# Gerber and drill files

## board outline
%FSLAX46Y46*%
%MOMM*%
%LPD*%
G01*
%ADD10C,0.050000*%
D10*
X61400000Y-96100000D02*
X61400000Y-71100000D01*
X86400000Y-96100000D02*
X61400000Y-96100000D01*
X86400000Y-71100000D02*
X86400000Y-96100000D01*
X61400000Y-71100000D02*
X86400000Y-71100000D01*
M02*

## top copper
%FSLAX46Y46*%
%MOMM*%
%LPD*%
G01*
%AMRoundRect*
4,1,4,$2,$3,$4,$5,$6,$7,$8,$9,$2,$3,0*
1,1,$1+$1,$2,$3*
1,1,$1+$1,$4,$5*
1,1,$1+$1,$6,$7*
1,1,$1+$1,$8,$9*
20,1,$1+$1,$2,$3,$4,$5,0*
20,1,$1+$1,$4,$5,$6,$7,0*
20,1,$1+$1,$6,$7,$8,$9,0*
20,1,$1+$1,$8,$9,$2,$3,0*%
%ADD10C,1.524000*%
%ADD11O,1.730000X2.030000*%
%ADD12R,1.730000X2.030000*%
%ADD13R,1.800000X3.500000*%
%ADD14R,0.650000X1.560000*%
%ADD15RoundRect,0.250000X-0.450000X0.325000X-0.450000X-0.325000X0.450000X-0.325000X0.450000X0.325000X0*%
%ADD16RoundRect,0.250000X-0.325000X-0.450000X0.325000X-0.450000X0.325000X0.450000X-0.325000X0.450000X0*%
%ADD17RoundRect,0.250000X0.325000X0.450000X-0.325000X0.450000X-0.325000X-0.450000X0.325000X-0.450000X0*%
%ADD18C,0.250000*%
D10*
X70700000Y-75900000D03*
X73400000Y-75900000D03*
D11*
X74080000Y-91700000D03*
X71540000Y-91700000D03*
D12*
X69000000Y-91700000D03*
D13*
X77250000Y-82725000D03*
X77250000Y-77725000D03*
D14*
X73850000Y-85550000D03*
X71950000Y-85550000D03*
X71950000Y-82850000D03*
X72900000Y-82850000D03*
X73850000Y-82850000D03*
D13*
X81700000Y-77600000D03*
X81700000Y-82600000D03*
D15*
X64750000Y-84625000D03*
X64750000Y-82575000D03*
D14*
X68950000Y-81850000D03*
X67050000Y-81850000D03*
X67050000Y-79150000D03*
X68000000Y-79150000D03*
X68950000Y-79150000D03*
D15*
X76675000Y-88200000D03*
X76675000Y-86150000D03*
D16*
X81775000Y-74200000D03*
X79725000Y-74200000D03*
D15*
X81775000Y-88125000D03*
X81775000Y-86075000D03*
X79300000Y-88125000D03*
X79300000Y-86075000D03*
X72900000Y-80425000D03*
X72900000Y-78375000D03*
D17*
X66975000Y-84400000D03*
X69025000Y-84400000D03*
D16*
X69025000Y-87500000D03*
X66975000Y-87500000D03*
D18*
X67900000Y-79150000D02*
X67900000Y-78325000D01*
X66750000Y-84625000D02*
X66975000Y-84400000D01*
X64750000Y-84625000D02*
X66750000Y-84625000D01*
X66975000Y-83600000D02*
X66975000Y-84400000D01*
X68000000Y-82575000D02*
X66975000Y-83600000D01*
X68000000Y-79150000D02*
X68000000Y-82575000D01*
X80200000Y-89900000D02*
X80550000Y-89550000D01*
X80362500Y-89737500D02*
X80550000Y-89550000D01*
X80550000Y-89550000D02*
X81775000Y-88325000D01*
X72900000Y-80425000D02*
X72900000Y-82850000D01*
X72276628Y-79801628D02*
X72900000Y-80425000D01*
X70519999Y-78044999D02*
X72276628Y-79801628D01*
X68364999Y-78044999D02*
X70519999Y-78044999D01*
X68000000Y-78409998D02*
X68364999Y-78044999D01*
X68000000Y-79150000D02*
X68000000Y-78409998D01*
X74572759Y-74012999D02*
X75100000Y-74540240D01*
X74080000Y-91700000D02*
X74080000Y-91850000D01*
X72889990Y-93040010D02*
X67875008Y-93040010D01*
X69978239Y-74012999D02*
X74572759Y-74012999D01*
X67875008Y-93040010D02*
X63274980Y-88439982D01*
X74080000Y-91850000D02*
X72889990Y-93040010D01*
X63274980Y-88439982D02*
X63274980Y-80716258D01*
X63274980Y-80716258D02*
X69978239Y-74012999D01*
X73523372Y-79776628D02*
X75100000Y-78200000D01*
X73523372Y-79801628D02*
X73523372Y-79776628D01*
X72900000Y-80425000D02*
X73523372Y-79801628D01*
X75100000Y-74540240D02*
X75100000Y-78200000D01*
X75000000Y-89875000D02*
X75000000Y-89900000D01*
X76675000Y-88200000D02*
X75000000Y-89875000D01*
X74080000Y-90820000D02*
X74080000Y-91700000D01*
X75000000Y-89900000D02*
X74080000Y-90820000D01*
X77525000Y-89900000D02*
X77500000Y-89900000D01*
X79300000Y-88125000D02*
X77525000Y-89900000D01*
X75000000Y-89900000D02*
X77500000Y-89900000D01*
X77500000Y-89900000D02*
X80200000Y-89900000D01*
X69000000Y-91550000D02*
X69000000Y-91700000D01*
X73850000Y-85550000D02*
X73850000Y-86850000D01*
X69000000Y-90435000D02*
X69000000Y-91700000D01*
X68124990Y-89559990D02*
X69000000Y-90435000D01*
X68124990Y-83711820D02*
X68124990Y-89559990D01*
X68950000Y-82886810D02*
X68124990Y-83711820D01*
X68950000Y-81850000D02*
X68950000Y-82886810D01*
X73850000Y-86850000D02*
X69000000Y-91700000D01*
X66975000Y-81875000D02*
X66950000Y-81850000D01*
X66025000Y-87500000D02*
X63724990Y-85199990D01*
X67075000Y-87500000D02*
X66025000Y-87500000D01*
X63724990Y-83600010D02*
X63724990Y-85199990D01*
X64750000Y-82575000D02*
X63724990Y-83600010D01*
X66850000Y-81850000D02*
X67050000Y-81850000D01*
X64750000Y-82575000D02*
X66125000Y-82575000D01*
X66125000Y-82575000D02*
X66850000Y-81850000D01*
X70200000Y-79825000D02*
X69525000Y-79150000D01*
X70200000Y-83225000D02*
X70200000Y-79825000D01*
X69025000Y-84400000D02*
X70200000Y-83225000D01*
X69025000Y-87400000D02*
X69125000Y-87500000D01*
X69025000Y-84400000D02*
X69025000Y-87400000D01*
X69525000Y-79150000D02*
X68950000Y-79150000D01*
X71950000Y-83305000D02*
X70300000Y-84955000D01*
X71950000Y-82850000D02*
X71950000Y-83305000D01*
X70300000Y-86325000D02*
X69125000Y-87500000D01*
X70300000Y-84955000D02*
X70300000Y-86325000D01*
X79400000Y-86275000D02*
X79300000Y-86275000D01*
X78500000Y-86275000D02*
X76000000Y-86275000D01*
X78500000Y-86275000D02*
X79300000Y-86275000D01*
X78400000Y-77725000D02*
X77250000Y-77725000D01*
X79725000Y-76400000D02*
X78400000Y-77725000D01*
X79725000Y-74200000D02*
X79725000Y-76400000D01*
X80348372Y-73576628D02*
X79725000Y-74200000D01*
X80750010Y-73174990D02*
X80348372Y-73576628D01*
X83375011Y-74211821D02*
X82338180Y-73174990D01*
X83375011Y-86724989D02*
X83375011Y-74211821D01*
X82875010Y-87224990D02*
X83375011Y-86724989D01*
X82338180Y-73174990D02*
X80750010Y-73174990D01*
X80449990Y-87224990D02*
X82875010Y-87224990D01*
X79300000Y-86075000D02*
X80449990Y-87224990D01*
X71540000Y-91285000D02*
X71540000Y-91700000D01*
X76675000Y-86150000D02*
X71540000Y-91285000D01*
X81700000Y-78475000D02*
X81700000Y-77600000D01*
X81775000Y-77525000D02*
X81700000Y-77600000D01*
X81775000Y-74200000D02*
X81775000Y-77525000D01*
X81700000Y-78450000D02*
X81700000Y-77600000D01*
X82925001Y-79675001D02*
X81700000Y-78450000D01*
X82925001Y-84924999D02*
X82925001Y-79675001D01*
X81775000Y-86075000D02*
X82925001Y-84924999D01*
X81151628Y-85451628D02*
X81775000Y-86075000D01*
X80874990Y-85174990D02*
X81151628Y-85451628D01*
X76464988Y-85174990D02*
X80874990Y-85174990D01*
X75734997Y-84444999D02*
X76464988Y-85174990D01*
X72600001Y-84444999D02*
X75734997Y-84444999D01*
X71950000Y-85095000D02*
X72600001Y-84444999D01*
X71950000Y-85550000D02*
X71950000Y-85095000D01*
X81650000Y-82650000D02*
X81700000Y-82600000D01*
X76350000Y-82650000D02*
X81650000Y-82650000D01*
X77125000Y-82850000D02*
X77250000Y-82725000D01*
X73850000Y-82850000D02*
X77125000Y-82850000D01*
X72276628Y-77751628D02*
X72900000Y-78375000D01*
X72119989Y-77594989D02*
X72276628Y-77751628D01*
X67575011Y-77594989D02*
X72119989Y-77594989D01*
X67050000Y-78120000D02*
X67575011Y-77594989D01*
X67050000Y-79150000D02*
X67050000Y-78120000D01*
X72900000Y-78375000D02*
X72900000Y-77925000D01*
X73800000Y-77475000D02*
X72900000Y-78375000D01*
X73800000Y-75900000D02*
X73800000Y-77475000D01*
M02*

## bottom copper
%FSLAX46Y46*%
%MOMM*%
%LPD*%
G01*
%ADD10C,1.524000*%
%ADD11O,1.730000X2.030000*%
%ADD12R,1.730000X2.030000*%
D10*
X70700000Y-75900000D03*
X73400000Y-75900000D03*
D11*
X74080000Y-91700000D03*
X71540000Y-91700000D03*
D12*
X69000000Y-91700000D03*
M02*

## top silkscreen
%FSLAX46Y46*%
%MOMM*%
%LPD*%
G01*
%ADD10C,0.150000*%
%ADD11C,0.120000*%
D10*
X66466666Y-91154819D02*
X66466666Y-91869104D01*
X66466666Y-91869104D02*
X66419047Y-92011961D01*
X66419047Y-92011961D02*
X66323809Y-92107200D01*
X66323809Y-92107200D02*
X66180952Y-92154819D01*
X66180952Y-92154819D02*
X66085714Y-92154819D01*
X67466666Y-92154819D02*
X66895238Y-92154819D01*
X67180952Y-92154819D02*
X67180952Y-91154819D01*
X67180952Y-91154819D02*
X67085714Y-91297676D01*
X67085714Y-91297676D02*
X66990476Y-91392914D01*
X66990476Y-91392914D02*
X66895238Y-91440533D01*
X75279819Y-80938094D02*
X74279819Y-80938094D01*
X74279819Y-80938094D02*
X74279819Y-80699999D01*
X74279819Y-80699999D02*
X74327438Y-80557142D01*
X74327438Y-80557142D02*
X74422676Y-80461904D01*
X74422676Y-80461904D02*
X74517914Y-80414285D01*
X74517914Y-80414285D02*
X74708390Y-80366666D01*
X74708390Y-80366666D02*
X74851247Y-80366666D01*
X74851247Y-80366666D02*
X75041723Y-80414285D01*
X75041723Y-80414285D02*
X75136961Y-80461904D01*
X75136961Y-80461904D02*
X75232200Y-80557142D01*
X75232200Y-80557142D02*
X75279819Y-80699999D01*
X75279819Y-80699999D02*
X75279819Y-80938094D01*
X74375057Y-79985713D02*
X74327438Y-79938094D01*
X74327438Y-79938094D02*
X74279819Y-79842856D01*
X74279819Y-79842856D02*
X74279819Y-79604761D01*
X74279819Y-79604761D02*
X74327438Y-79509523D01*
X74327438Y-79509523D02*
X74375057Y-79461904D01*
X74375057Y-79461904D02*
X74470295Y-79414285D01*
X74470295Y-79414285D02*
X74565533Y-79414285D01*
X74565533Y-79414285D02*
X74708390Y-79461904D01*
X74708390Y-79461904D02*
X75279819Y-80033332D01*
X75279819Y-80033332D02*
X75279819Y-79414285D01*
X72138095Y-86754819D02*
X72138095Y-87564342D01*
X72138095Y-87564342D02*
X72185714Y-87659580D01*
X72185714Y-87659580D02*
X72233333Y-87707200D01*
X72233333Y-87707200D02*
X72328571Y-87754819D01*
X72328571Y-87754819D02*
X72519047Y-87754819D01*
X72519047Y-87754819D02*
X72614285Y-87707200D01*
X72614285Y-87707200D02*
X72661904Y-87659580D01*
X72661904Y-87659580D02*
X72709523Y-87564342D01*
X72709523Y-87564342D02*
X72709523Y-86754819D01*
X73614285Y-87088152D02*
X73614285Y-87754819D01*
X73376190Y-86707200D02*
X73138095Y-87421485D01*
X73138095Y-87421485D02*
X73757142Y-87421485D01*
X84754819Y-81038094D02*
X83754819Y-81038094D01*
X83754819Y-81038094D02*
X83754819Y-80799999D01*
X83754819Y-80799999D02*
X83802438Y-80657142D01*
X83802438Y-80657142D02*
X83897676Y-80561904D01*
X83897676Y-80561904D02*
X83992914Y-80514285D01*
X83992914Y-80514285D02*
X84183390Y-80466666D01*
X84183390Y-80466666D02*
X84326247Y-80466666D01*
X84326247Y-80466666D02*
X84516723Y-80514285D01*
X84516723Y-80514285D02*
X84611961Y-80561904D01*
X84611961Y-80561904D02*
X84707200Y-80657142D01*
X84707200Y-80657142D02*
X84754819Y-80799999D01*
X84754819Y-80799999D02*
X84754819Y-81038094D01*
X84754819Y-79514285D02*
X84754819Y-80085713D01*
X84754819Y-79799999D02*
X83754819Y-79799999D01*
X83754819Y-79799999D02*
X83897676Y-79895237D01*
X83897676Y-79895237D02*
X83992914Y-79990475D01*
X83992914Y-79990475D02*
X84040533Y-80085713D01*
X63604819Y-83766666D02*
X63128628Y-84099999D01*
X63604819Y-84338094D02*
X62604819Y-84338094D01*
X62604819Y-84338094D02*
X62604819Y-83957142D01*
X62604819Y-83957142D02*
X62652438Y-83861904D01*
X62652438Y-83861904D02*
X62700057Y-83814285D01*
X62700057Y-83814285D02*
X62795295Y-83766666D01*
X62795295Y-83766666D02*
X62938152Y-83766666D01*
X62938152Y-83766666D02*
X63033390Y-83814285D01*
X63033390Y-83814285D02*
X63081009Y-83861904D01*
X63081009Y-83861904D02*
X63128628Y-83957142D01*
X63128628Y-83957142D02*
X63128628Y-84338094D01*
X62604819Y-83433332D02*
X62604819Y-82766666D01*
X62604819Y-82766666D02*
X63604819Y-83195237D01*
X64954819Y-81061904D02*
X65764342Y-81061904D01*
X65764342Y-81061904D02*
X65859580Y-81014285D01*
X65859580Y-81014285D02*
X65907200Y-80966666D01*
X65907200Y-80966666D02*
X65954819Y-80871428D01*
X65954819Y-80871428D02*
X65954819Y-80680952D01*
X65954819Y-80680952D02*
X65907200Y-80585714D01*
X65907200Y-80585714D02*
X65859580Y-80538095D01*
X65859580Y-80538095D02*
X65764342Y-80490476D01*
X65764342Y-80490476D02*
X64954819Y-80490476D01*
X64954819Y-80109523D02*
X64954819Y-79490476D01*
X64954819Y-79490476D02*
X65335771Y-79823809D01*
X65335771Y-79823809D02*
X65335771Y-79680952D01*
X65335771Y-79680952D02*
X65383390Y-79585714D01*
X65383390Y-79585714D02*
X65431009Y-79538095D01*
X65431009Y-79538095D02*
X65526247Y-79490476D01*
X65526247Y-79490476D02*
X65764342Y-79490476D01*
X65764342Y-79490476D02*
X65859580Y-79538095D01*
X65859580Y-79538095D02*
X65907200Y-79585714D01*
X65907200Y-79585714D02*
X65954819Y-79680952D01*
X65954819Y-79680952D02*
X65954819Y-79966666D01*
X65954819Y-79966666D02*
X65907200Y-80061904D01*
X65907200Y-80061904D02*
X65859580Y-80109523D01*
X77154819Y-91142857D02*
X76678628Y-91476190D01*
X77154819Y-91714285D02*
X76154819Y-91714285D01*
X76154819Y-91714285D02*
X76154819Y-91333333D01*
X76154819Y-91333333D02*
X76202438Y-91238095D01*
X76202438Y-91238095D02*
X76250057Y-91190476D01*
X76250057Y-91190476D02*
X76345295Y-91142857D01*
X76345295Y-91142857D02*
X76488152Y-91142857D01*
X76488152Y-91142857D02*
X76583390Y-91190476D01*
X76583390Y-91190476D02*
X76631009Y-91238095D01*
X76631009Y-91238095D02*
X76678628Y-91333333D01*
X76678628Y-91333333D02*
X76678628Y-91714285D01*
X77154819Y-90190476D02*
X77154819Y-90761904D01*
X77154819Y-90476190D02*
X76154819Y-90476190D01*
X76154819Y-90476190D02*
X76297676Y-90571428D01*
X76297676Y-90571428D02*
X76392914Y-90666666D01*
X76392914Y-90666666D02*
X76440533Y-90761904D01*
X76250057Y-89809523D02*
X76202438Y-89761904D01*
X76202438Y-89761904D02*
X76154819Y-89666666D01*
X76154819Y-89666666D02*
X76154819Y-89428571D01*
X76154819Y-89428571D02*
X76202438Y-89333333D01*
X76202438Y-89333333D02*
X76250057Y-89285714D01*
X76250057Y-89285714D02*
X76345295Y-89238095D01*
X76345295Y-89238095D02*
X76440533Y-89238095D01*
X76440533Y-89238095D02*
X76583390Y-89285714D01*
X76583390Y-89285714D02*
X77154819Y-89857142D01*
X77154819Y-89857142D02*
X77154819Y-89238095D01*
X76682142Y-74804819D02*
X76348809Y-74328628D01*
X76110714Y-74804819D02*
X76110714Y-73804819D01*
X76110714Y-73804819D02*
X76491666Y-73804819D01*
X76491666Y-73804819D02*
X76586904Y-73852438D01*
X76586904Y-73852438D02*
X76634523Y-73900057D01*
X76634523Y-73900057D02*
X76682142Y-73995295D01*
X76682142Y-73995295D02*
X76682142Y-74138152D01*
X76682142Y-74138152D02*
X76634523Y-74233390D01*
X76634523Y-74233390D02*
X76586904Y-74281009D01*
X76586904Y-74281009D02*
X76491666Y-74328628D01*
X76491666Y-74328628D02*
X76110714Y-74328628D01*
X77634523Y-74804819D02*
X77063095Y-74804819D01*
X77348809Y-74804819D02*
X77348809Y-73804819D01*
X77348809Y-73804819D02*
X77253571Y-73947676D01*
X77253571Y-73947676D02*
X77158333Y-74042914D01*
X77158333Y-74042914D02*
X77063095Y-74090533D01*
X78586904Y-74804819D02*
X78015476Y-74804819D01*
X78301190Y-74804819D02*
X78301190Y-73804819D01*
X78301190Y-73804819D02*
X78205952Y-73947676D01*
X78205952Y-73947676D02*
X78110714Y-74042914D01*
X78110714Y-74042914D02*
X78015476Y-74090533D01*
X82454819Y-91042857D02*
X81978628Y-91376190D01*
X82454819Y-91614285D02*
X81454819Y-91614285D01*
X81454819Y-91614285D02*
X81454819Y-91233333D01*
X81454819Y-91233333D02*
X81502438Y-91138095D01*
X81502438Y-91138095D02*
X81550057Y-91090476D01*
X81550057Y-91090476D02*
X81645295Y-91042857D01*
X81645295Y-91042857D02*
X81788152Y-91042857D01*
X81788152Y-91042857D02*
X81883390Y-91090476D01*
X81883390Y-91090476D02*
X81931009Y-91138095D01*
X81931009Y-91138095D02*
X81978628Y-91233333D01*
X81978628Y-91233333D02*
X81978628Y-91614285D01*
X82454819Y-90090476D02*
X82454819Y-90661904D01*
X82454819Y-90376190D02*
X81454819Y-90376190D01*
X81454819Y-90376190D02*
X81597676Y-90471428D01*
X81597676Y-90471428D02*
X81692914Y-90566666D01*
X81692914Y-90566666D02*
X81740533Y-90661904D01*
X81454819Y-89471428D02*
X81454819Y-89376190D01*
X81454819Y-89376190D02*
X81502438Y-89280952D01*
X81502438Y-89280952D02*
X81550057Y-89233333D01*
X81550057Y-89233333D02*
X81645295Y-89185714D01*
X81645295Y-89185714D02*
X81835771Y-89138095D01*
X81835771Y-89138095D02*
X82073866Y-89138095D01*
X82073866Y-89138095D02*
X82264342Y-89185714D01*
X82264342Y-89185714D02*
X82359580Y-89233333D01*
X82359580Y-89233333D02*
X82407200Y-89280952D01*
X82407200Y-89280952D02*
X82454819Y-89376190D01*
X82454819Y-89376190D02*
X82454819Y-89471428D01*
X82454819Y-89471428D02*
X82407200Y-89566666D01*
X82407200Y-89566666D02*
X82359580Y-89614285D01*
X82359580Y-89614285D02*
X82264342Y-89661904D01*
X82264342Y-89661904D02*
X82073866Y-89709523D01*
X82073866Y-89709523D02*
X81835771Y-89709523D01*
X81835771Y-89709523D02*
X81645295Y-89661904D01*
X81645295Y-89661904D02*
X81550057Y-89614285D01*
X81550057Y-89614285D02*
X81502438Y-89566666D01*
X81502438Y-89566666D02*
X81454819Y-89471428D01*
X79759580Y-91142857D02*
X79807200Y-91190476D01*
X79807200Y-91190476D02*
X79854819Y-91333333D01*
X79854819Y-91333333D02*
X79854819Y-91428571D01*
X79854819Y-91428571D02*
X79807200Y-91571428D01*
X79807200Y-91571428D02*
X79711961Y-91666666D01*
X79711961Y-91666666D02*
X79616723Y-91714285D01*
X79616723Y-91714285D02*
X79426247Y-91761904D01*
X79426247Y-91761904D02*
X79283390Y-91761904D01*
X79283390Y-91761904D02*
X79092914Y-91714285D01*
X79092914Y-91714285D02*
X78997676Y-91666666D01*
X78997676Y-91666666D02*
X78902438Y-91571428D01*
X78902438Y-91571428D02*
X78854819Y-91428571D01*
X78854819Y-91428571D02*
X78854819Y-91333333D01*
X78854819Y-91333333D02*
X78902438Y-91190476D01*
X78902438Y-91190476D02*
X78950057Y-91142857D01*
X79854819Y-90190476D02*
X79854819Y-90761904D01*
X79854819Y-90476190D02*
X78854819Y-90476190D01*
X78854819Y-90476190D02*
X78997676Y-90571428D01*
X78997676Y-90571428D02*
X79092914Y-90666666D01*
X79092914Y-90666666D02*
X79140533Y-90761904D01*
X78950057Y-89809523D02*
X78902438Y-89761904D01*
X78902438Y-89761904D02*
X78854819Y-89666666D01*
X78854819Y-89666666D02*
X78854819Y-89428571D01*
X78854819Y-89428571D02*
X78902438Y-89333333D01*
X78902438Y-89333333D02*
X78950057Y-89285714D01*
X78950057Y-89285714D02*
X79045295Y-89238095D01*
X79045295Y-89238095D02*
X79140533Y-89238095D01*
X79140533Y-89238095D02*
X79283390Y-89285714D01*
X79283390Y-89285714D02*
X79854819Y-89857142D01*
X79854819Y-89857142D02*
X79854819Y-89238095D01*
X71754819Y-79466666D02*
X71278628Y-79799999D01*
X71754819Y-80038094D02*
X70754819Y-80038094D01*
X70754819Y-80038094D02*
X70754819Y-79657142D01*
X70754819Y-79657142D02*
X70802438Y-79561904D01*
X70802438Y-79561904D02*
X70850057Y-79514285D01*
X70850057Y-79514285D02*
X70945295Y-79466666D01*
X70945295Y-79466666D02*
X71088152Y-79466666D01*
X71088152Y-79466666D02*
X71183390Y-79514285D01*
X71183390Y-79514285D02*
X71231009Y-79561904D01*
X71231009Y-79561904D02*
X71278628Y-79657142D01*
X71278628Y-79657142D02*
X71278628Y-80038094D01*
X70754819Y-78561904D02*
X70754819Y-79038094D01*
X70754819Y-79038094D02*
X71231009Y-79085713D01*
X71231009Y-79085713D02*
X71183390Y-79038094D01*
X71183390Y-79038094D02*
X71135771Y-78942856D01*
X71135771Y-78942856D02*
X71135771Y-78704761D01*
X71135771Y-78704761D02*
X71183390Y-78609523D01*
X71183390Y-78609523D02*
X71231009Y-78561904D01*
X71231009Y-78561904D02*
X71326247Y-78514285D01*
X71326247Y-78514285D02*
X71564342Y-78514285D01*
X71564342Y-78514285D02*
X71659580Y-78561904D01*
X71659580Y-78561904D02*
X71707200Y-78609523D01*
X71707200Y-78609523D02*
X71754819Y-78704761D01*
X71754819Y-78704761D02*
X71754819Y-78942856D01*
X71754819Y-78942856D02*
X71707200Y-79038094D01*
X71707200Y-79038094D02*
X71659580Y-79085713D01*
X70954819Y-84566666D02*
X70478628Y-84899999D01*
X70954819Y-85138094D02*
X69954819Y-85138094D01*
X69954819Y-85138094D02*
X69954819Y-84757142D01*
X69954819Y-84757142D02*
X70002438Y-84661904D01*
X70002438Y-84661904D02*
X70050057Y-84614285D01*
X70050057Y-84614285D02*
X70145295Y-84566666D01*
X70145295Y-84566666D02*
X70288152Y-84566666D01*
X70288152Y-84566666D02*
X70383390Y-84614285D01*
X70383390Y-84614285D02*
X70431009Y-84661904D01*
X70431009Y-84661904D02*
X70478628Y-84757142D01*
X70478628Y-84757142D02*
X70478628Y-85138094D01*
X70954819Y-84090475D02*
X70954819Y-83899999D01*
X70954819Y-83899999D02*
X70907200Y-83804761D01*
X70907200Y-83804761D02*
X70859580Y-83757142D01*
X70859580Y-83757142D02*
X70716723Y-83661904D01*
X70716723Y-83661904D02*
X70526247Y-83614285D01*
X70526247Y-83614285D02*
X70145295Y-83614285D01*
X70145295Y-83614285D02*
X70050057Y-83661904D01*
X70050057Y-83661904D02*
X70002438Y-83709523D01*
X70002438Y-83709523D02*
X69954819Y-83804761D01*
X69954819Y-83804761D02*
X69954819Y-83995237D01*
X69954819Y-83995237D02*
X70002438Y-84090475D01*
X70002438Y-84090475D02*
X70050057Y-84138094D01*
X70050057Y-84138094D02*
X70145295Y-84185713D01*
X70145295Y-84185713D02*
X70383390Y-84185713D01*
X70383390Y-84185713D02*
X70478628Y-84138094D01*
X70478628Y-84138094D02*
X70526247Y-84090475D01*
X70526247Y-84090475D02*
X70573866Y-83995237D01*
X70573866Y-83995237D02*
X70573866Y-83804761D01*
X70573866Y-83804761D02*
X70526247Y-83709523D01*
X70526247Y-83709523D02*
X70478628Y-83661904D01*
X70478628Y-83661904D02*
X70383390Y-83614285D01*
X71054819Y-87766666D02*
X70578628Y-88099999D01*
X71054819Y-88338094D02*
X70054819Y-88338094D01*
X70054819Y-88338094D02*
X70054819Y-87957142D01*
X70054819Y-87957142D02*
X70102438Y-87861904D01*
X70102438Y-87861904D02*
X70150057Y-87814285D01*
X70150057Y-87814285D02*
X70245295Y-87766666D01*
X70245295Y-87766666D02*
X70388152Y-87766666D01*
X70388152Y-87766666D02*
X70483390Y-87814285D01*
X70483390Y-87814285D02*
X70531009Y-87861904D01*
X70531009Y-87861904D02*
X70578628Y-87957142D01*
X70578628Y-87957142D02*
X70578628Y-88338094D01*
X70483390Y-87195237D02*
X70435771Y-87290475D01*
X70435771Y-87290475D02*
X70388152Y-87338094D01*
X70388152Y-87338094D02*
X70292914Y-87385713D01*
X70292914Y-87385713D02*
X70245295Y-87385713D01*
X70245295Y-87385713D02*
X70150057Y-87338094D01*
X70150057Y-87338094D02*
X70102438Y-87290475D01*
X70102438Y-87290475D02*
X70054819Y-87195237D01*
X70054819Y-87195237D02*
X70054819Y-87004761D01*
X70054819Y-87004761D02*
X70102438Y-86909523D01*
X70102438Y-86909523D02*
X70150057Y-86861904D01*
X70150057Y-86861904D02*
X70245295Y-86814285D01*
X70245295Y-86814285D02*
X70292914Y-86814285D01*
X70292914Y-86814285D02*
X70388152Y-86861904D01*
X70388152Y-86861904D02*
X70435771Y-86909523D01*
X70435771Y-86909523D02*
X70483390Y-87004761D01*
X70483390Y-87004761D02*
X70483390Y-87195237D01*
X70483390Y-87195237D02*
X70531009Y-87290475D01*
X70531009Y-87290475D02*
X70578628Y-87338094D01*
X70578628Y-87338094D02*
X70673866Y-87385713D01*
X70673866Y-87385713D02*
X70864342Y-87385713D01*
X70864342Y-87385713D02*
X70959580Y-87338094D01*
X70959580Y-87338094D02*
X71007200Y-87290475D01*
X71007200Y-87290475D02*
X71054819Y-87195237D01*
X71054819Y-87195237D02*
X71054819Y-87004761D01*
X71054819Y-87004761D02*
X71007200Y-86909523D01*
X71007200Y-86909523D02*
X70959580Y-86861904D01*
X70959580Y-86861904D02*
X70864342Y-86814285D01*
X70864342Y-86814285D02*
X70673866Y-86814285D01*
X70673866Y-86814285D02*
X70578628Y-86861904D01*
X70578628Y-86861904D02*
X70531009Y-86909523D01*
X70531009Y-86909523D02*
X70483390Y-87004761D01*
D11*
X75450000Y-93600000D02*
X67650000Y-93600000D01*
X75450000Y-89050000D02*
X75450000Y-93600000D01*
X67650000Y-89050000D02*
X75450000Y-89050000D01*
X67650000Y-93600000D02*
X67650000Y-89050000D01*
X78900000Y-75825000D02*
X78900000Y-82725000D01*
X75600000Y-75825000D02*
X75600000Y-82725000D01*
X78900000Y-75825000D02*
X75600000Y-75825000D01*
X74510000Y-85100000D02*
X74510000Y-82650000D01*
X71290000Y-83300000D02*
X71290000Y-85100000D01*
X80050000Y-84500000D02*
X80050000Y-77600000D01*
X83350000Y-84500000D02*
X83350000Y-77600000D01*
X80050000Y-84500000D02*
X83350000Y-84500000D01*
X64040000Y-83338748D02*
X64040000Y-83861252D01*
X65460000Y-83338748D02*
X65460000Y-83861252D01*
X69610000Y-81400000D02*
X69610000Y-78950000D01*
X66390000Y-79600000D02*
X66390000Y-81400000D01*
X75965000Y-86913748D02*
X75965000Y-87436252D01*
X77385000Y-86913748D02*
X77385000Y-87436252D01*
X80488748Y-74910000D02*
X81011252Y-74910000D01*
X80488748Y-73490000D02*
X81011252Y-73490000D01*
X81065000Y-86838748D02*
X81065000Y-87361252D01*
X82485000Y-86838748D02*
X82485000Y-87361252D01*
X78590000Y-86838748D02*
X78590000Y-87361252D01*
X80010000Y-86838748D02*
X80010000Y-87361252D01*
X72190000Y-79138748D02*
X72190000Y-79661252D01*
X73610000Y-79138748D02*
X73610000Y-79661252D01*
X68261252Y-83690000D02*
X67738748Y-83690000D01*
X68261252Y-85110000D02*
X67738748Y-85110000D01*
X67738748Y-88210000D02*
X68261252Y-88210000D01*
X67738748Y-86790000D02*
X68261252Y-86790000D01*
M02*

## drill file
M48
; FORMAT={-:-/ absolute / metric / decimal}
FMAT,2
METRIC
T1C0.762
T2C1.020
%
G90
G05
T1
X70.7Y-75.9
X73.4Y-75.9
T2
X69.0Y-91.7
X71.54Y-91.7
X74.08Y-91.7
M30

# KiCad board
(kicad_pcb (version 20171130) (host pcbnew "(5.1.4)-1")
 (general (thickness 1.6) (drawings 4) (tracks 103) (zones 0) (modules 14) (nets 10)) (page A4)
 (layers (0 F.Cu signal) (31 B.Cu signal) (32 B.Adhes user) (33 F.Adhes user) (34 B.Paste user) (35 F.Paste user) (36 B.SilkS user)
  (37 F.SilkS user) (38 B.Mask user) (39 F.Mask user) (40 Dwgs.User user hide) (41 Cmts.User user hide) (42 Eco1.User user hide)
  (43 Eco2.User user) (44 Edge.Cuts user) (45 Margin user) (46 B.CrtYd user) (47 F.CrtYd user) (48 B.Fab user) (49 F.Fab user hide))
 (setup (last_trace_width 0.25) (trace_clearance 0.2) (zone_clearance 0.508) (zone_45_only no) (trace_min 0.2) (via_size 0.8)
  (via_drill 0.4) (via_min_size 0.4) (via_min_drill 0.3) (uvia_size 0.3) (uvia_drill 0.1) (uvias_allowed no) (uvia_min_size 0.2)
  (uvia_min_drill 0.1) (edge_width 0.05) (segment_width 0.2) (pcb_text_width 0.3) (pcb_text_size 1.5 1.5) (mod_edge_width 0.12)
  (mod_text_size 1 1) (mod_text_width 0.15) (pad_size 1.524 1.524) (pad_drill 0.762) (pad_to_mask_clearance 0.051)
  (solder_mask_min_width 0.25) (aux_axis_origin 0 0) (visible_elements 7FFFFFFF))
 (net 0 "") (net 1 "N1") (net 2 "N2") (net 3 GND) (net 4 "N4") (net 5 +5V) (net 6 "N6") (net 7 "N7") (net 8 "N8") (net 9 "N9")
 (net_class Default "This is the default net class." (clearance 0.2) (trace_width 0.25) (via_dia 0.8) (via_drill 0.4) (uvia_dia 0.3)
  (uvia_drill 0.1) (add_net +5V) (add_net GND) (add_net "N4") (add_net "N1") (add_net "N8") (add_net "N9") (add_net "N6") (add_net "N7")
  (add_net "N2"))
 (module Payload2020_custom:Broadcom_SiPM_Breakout (layer B.Cu) (at 72.5 81.8 90)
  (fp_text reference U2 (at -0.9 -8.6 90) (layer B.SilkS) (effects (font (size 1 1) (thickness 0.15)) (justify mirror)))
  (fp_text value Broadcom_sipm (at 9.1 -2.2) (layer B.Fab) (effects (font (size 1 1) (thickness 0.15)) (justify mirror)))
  (pad 1 thru_hole circle (at 5.9 -1.8 90) (size 1.524 1.524) (drill 0.762) (layers *.Cu *.Mask) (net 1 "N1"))
  (pad 2 thru_hole circle (at 5.9 0.9 90) (size 1.524 1.524) (drill 0.762) (layers *.Cu *.Mask) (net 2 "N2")))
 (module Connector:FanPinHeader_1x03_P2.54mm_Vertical (layer F.Cu) (at 69 91.7)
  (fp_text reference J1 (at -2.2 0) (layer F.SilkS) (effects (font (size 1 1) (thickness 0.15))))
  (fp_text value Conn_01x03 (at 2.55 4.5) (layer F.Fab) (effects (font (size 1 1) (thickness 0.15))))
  (fp_line (start 6.45 1.9) (end -1.35 1.9) (layer F.SilkS) (width 0.12))
  (fp_line (start 6.45 -2.65) (end 6.45 1.9) (layer F.SilkS) (width 0.12))
  (fp_line (start -1.35 -2.65) (end 6.45 -2.65) (layer F.SilkS) (width 0.12))
  (fp_line (start -1.35 1.9) (end -1.35 -2.65) (layer F.SilkS) (width 0.12))
  (pad 3 thru_hole oval (at 5.08 0 90) (size 2.03 1.73) (drill 1.02) (layers *.Cu *.Mask) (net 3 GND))
  (pad 2 thru_hole oval (at 2.54 0 90) (size 2.03 1.73) (drill 1.02) (layers *.Cu *.Mask) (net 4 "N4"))
  (pad 1 thru_hole rect (at 0 0 90) (size 2.03 1.73) (drill 1.02) (layers *.Cu *.Mask) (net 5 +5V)))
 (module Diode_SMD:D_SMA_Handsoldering (layer F.Cu) (at 77.25 80.225 270)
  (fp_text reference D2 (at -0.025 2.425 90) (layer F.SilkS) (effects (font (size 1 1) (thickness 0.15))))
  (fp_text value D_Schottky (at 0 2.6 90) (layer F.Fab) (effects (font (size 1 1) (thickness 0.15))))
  (fp_line (start -4.4 -1.65) (end 2.5 -1.65) (layer F.SilkS) (width 0.12))
  (fp_line (start -4.4 1.65) (end 2.5 1.65) (layer F.SilkS) (width 0.12))
  (fp_line (start -4.4 -1.65) (end -4.4 1.65) (layer F.SilkS) (width 0.12))
  (pad 2 smd rect (at 2.5 0 270) (size 3.5 1.8) (layers F.Cu F.Paste F.Mask) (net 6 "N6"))
  (pad 1 smd rect (at -2.5 0 270) (size 3.5 1.8) (layers F.Cu F.Paste F.Mask) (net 4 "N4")))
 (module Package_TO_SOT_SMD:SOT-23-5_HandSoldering (layer F.Cu) (at 72.9 84.2 270)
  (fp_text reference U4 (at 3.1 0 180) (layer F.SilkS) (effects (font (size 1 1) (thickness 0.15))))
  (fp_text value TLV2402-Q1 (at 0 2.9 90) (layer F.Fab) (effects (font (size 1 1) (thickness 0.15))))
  (fp_line (start 0.9 -1.61) (end -1.55 -1.61) (layer F.SilkS) (width 0.12))
  (fp_line (start -0.9 1.61) (end 0.9 1.61) (layer F.SilkS) (width 0.12))
  (pad 5 smd rect (at 1.35 -0.95 270) (size 1.56 0.65) (layers F.Cu F.Paste F.Mask) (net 5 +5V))
  (pad 4 smd rect (at 1.35 0.95 270) (size 1.56 0.65) (layers F.Cu F.Paste F.Mask) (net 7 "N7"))
  (pad 3 smd rect (at -1.35 0.95 270) (size 1.56 0.65) (layers F.Cu F.Paste F.Mask) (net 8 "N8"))
  (pad 2 smd rect (at -1.35 0 270) (size 1.56 0.65) (layers F.Cu F.Paste F.Mask) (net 3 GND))
  (pad 1 smd rect (at -1.35 -0.95 270) (size 1.56 0.65) (layers F.Cu F.Paste F.Mask) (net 6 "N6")))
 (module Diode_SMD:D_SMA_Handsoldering (layer F.Cu) (at 81.7 80.1 90)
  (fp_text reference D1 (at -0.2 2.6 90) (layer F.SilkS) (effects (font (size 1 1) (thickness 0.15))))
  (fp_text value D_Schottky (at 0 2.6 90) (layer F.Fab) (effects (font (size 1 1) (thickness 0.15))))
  (fp_line (start -4.4 -1.65) (end 2.5 -1.65) (layer F.SilkS) (width 0.12))
  (fp_line (start -4.4 1.65) (end 2.5 1.65) (layer F.SilkS) (width 0.12))
  (fp_line (start -4.4 -1.65) (end -4.4 1.65) (layer F.SilkS) (width 0.12))
  (pad 2 smd rect (at 2.5 0 90) (size 3.5 1.8) (layers F.Cu F.Paste F.Mask) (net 7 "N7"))
  (pad 1 smd rect (at -2.5 0 90) (size 3.5 1.8) (layers F.Cu F.Paste F.Mask) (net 6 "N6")))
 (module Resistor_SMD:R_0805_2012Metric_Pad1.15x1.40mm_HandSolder (layer F.Cu) (at 64.75 83.6 270)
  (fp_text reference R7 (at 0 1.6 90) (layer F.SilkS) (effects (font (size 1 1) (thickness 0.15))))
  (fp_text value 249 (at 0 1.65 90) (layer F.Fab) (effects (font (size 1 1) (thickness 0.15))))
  (fp_line (start -0.261252 0.71) (end 0.261252 0.71) (layer F.SilkS) (width 0.12))
  (fp_line (start -0.261252 -0.71) (end 0.261252 -0.71) (layer F.SilkS) (width 0.12))
  (pad 2 smd roundrect (at 1.025 0 270) (size 1.15 1.4) (layers F.Cu F.Paste F.Mask) (roundrect_rratio 0.217391) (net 3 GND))
  (pad 1 smd roundrect (at -1.025 0 270) (size 1.15 1.4) (layers F.Cu F.Paste F.Mask) (roundrect_rratio 0.217391) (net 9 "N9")))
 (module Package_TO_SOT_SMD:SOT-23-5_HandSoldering (layer F.Cu) (at 68 80.5 270)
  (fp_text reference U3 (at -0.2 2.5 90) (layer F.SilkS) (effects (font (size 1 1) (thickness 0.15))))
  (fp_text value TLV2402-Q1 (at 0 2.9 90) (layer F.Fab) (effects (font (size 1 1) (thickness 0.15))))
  (fp_line (start 0.9 -1.61) (end -1.55 -1.61) (layer F.SilkS) (width 0.12))
  (fp_line (start -0.9 1.61) (end 0.9 1.61) (layer F.SilkS) (width 0.12))
  (pad 5 smd rect (at 1.35 -0.95 270) (size 1.56 0.65) (layers F.Cu F.Paste F.Mask) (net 5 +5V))
  (pad 4 smd rect (at 1.35 0.95 270) (size 1.56 0.65) (layers F.Cu F.Paste F.Mask) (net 9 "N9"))
  (pad 3 smd rect (at -1.35 0.95 270) (size 1.56 0.65) (layers F.Cu F.Paste F.Mask) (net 2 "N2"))
  (pad 2 smd rect (at -1.35 0 270) (size 1.56 0.65) (layers F.Cu F.Paste F.Mask) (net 3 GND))
  (pad 1 smd rect (at -1.35 -0.95 270) (size 1.56 0.65) (layers F.Cu F.Paste F.Mask) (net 8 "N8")))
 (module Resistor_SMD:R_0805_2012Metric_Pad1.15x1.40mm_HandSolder (layer F.Cu) (at 76.675 87.175 270)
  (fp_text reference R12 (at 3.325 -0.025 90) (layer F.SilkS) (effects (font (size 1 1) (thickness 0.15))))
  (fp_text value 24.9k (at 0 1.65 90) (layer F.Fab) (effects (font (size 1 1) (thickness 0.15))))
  (fp_line (start -0.261252 0.71) (end 0.261252 0.71) (layer F.SilkS) (width 0.12))
  (fp_line (start -0.261252 -0.71) (end 0.261252 -0.71) (layer F.SilkS) (width 0.12))
  (pad 2 smd roundrect (at 1.025 0 270) (size 1.15 1.4) (layers F.Cu F.Paste F.Mask) (roundrect_rratio 0.217391) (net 3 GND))
  (pad 1 smd roundrect (at -1.025 0 270) (size 1.15 1.4) (layers F.Cu F.Paste F.Mask) (roundrect_rratio 0.217391) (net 4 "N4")))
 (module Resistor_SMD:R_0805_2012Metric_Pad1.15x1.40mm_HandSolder (layer F.Cu) (at 80.75 74.2)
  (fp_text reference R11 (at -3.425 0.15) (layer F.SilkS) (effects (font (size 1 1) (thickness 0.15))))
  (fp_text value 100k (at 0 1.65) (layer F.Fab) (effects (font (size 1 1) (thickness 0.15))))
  (fp_line (start -0.261252 0.71) (end 0.261252 0.71) (layer F.SilkS) (width 0.12))
  (fp_line (start -0.261252 -0.71) (end 0.261252 -0.71) (layer F.SilkS) (width 0.12))
  (pad 2 smd roundrect (at 1.025 0) (size 1.15 1.4) (layers F.Cu F.Paste F.Mask) (roundrect_rratio 0.217391) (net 7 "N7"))
  (pad 1 smd roundrect (at -1.025 0) (size 1.15 1.4) (layers F.Cu F.Paste F.Mask) (roundrect_rratio 0.217391) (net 4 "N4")))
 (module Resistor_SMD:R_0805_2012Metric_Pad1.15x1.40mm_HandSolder (layer F.Cu) (at 81.775 87.1 270)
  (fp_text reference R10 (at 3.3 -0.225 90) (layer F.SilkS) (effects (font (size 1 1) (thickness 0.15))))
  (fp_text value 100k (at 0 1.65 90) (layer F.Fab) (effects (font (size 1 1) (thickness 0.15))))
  (fp_line (start -0.261252 0.71) (end 0.261252 0.71) (layer F.SilkS) (width 0.12))
  (fp_line (start -0.261252 -0.71) (end 0.261252 -0.71) (layer F.SilkS) (width 0.12))
  (pad 2 smd roundrect (at 1.025 0 270) (size 1.15 1.4) (layers F.Cu F.Paste F.Mask) (roundrect_rratio 0.217391) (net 3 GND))
  (pad 1 smd roundrect (at -1.025 0 270) (size 1.15 1.4) (layers F.Cu F.Paste F.Mask) (roundrect_rratio 0.217391) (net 7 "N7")))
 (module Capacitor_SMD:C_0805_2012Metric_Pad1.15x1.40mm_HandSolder (layer F.Cu) (at 79.3 87.1 270)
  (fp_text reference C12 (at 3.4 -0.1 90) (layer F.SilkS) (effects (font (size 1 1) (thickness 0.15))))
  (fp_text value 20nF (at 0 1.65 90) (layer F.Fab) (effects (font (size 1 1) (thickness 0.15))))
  (fp_line (start -0.261252 0.71) (end 0.261252 0.71) (layer F.SilkS) (width 0.12))
  (fp_line (start -0.261252 -0.71) (end 0.261252 -0.71) (layer F.SilkS) (width 0.12))
  (pad 2 smd roundrect (at 1.025 0 270) (size 1.15 1.4) (layers F.Cu F.Paste F.Mask) (roundrect_rratio 0.217391) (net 3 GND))
  (pad 1 smd roundrect (at -1.025 0 270) (size 1.15 1.4) (layers F.Cu F.Paste F.Mask) (roundrect_rratio 0.217391) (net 4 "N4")))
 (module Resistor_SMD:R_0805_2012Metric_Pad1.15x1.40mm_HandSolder (layer F.Cu) (at 72.9 79.4 270)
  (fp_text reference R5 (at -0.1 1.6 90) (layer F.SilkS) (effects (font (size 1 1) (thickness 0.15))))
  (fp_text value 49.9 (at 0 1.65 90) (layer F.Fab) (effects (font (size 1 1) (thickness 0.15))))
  (fp_line (start -0.261252 0.71) (end 0.261252 0.71) (layer F.SilkS) (width 0.12))
  (fp_line (start -0.261252 -0.71) (end 0.261252 -0.71) (layer F.SilkS) (width 0.12))
  (pad 2 smd roundrect (at 1.025 0 270) (size 1.15 1.4) (layers F.Cu F.Paste F.Mask) (roundrect_rratio 0.217391) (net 3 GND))
  (pad 1 smd roundrect (at -1.025 0 270) (size 1.15 1.4) (layers F.Cu F.Paste F.Mask) (roundrect_rratio 0.217391) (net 2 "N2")))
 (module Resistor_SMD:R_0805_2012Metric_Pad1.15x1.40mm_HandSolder (layer F.Cu) (at 68 84.4 180)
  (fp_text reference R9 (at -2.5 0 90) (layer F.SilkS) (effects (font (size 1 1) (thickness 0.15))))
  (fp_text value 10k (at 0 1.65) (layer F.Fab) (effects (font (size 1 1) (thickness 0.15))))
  (fp_line (start -0.261252 0.71) (end 0.261252 0.71) (layer F.SilkS) (width 0.12))
  (fp_line (start -0.261252 -0.71) (end 0.261252 -0.71) (layer F.SilkS) (width 0.12))
  (pad 2 smd roundrect (at 1.025 0 180) (size 1.15 1.4) (layers F.Cu F.Paste F.Mask) (roundrect_rratio 0.217391) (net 3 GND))
  (pad 1 smd roundrect (at -1.025 0 180) (size 1.15 1.4) (layers F.Cu F.Paste F.Mask) (roundrect_rratio 0.217391) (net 8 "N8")))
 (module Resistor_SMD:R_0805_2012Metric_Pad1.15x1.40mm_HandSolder (layer F.Cu) (at 68 87.5)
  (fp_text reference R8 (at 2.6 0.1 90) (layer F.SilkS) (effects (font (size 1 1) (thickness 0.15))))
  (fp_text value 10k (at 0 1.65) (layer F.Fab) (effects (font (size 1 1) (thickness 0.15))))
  (fp_line (start -0.261252 0.71) (end 0.261252 0.71) (layer F.SilkS) (width 0.12))
  (fp_line (start -0.261252 -0.71) (end 0.261252 -0.71) (layer F.SilkS) (width 0.12))
  (pad 2 smd roundrect (at 1.025 0) (size 1.15 1.4) (layers F.Cu F.Paste F.Mask) (roundrect_rratio 0.217391) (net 8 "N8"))
  (pad 1 smd roundrect (at -1.025 0) (size 1.15 1.4) (layers F.Cu F.Paste F.Mask) (roundrect_rratio 0.217391) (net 9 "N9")))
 (gr_line (start 61.4 96.1) (end 61.4 71.1) (layer Edge.Cuts) (width 0.05))
 (gr_line (start 86.4 96.1) (end 61.4 96.1) (layer Edge.Cuts) (width 0.05))
 (gr_line (start 86.4 71.1) (end 86.4 96.1) (layer Edge.Cuts) (width 0.05))
 (gr_line (start 61.4 71.1) (end 86.4 71.1) (layer Edge.Cuts) (width 0.05))
 (segment (start 67.9 79.15) (end 67.9 78.325) (width 0.25) (layer F.Cu) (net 3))
 (segment (start 66.75 84.625) (end 66.975 84.4) (width 0.25) (layer F.Cu) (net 3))
 (segment (start 64.75 84.625) (end 66.75 84.625) (width 0.25) (layer F.Cu) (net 3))
 (segment (start 66.975 83.6) (end 66.975 84.4) (width 0.25) (layer F.Cu) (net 3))
 (segment (start 68 82.575) (end 66.975 83.6) (width 0.25) (layer F.Cu) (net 3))
 (segment (start 68 79.15) (end 68 82.575) (width 0.25) (layer F.Cu) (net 3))
 (segment (start 80.2 89.9) (end 80.55 89.55) (width 0.25) (layer F.Cu) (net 3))
 (segment (start 80.3625 89.7375) (end 80.55 89.55) (width 0.25) (layer F.Cu) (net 3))
 (segment (start 80.55 89.55) (end 81.775 88.325) (width 0.25) (layer F.Cu) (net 3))
 (segment (start 72.9 80.425) (end 72.9 82.85) (width 0.25) (layer F.Cu) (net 3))
 (segment (start 72.276628 79.801628) (end 72.9 80.425) (width 0.25) (layer F.Cu) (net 3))
 (segment (start 70.519999 78.044999) (end 72.276628 79.801628) (width 0.25) (layer F.Cu) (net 3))
 (segment (start 68.364999 78.044999) (end 70.519999 78.044999) (width 0.25) (layer F.Cu) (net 3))
 (segment (start 68 78.409998) (end 68.364999 78.044999) (width 0.25) (layer F.Cu) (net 3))
 (segment (start 68 79.15) (end 68 78.409998) (width 0.25) (layer F.Cu) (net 3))
 (segment (start 74.572759 74.012999) (end 75.1 74.54024) (width 0.25) (layer F.Cu) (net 3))
 (segment (start 74.08 91.7) (end 74.08 91.85) (width 0.25) (layer F.Cu) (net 3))
 (segment (start 72.88999 93.04001) (end 67.875008 93.04001) (width 0.25) (layer F.Cu) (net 3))
 (segment (start 69.978239 74.012999) (end 74.572759 74.012999) (width 0.25) (layer F.Cu) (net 3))
 (segment (start 67.875008 93.04001) (end 63.27498 88.439982) (width 0.25) (layer F.Cu) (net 3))
 (segment (start 74.08 91.85) (end 72.88999 93.04001) (width 0.25) (layer F.Cu) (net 3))
 (segment (start 63.27498 88.439982) (end 63.27498 80.716258) (width 0.25) (layer F.Cu) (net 3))
 (segment (start 63.27498 80.716258) (end 69.978239 74.012999) (width 0.25) (layer F.Cu) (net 3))
 (segment (start 73.523372 79.776628) (end 75.1 78.2) (width 0.25) (layer F.Cu) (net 3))
 (segment (start 73.523372 79.801628) (end 73.523372 79.776628) (width 0.25) (layer F.Cu) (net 3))
 (segment (start 72.9 80.425) (end 73.523372 79.801628) (width 0.25) (layer F.Cu) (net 3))
 (segment (start 75.1 74.54024) (end 75.1 78.2) (width 0.25) (layer F.Cu) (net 3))
 (segment (start 75 89.875) (end 75 89.9) (width 0.25) (layer F.Cu) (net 3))
 (segment (start 76.675 88.2) (end 75 89.875) (width 0.25) (layer F.Cu) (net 3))
 (segment (start 74.08 90.82) (end 74.08 91.7) (width 0.25) (layer F.Cu) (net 3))
 (segment (start 75 89.9) (end 74.08 90.82) (width 0.25) (layer F.Cu) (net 3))
 (segment (start 77.525 89.9) (end 77.5 89.9) (width 0.25) (layer F.Cu) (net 3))
 (segment (start 79.3 88.125) (end 77.525 89.9) (width 0.25) (layer F.Cu) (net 3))
 (segment (start 75 89.9) (end 77.5 89.9) (width 0.25) (layer F.Cu) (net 3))
 (segment (start 77.5 89.9) (end 80.2 89.9) (width 0.25) (layer F.Cu) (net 3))
 (segment (start 69 91.55) (end 69 91.7) (width 0.25) (layer F.Cu) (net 5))
 (segment (start 73.85 85.55) (end 73.85 86.85) (width 0.25) (layer F.Cu) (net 5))
 (segment (start 69 90.435) (end 69 91.7) (width 0.25) (layer F.Cu) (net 5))
 (segment (start 68.12499 89.55999) (end 69 90.435) (width 0.25) (layer F.Cu) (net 5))
 (segment (start 68.12499 83.71182) (end 68.12499 89.55999) (width 0.25) (layer F.Cu) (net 5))
 (segment (start 68.95 82.88681) (end 68.12499 83.71182) (width 0.25) (layer F.Cu) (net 5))
 (segment (start 68.95 81.85) (end 68.95 82.88681) (width 0.25) (layer F.Cu) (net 5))
 (segment (start 73.85 86.85) (end 69 91.7) (width 0.25) (layer F.Cu) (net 5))
 (segment (start 66.975 81.875) (end 66.95 81.85) (width 0.25) (layer F.Cu) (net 9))
 (segment (start 66.025 87.5) (end 63.72499 85.19999) (width 0.25) (layer F.Cu) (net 9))
 (segment (start 67.075 87.5) (end 66.025 87.5) (width 0.25) (layer F.Cu) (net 9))
 (segment (start 63.72499 83.60001) (end 63.72499 85.19999) (width 0.25) (layer F.Cu) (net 9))
 (segment (start 64.75 82.575) (end 63.72499 83.60001) (width 0.25) (layer F.Cu) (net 9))
 (segment (start 66.85 81.85) (end 67.05 81.85) (width 0.25) (layer F.Cu) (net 9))
 (segment (start 64.75 82.575) (end 66.125 82.575) (width 0.25) (layer F.Cu) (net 9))
 (segment (start 66.125 82.575) (end 66.85 81.85) (width 0.25) (layer F.Cu) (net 9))
 (segment (start 70.2 79.825) (end 69.525 79.15) (width 0.25) (layer F.Cu) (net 8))
 (segment (start 70.2 83.225) (end 70.2 79.825) (width 0.25) (layer F.Cu) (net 8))
 (segment (start 69.025 84.4) (end 70.2 83.225) (width 0.25) (layer F.Cu) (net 8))
 (segment (start 69.025 87.4) (end 69.125 87.5) (width 0.25) (layer F.Cu) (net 8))
 (segment (start 69.025 84.4) (end 69.025 87.4) (width 0.25) (layer F.Cu) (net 8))
 (segment (start 69.525 79.15) (end 68.95 79.15) (width 0.25) (layer F.Cu) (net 8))
 (segment (start 71.95 83.305) (end 70.3 84.955) (width 0.25) (layer F.Cu) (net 8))
 (segment (start 71.95 82.85) (end 71.95 83.305) (width 0.25) (layer F.Cu) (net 8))
 (segment (start 70.3 86.325) (end 69.125 87.5) (width 0.25) (layer F.Cu) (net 8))
 (segment (start 70.3 84.955) (end 70.3 86.325) (width 0.25) (layer F.Cu) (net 8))
 (segment (start 79.4 86.275) (end 79.3 86.275) (width 0.25) (layer F.Cu) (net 4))
 (segment (start 78.5 86.275) (end 76 86.275) (width 0.25) (layer F.Cu) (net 4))
 (segment (start 78.5 86.275) (end 79.3 86.275) (width 0.25) (layer F.Cu) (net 4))
 (segment (start 78.4 77.725) (end 77.25 77.725) (width 0.25) (layer F.Cu) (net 4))
 (segment (start 79.725 76.4) (end 78.4 77.725) (width 0.25) (layer F.Cu) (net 4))
 (segment (start 79.725 74.2) (end 79.725 76.4) (width 0.25) (layer F.Cu) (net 4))
 (segment (start 80.348372 73.576628) (end 79.725 74.2) (width 0.25) (layer F.Cu) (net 4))
 (segment (start 80.75001 73.17499) (end 80.348372 73.576628) (width 0.25) (layer F.Cu) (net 4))
 (segment (start 83.375011 74.211821) (end 82.33818 73.17499) (width 0.25) (layer F.Cu) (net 4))
 (segment (start 83.375011 86.724989) (end 83.375011 74.211821) (width 0.25) (layer F.Cu) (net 4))
 (segment (start 82.87501 87.22499) (end 83.375011 86.724989) (width 0.25) (layer F.Cu) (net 4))
 (segment (start 82.33818 73.17499) (end 80.75001 73.17499) (width 0.25) (layer F.Cu) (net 4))
 (segment (start 80.44999 87.22499) (end 82.87501 87.22499) (width 0.25) (layer F.Cu) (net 4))
 (segment (start 79.3 86.075) (end 80.44999 87.22499) (width 0.25) (layer F.Cu) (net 4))
 (segment (start 71.54 91.285) (end 71.54 91.7) (width 0.25) (layer F.Cu) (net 4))
 (segment (start 76.675 86.15) (end 71.54 91.285) (width 0.25) (layer F.Cu) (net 4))
 (segment (start 81.7 78.475) (end 81.7 77.6) (width 0.25) (layer F.Cu) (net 7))
 (segment (start 81.775 77.525) (end 81.7 77.6) (width 0.25) (layer F.Cu) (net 7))
 (segment (start 81.775 74.2) (end 81.775 77.525) (width 0.25) (layer F.Cu) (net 7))
 (segment (start 81.7 78.45) (end 81.7 77.6) (width 0.25) (layer F.Cu) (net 7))
 (segment (start 82.925001 79.675001) (end 81.7 78.45) (width 0.25) (layer F.Cu) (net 7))
 (segment (start 82.925001 84.924999) (end 82.925001 79.675001) (width 0.25) (layer F.Cu) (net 7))
 (segment (start 81.775 86.075) (end 82.925001 84.924999) (width 0.25) (layer F.Cu) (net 7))
 (segment (start 81.151628 85.451628) (end 81.775 86.075) (width 0.25) (layer F.Cu) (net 7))
 (segment (start 80.87499 85.17499) (end 81.151628 85.451628) (width 0.25) (layer F.Cu) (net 7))
 (segment (start 76.464988 85.17499) (end 80.87499 85.17499) (width 0.25) (layer F.Cu) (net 7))
 (segment (start 75.734997 84.444999) (end 76.464988 85.17499) (width 0.25) (layer F.Cu) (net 7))
 (segment (start 72.600001 84.444999) (end 75.734997 84.444999) (width 0.25) (layer F.Cu) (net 7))
 (segment (start 71.95 85.095) (end 72.600001 84.444999) (width 0.25) (layer F.Cu) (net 7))
 (segment (start 71.95 85.55) (end 71.95 85.095) (width 0.25) (layer F.Cu) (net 7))
 (segment (start 81.65 82.65) (end 81.7 82.6) (width 0.25) (layer F.Cu) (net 6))
 (segment (start 76.35 82.65) (end 81.65 82.65) (width 0.25) (layer F.Cu) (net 6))
 (segment (start 77.125 82.85) (end 77.25 82.725) (width 0.25) (layer F.Cu) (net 6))
 (segment (start 73.85 82.85) (end 77.125 82.85) (width 0.25) (layer F.Cu) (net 6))
 (segment (start 72.276628 77.751628) (end 72.9 78.375) (width 0.25) (layer F.Cu) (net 2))
 (segment (start 72.119989 77.594989) (end 72.276628 77.751628) (width 0.25) (layer F.Cu) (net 2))
 (segment (start 67.575011 77.594989) (end 72.119989 77.594989) (width 0.25) (layer F.Cu) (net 2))
 (segment (start 67.05 78.12) (end 67.575011 77.594989) (width 0.25) (layer F.Cu) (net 2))
 (segment (start 67.05 79.15) (end 67.05 78.12) (width 0.25) (layer F.Cu) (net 2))
 (segment (start 72.9 78.375) (end 72.9 77.925) (width 0.25) (layer F.Cu) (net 2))
 (segment (start 73.8 77.475) (end 72.9 78.375) (width 0.25) (layer F.Cu) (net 2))
 (segment (start 73.8 75.9) (end 73.8 77.475) (width 0.25) (layer F.Cu) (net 2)))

